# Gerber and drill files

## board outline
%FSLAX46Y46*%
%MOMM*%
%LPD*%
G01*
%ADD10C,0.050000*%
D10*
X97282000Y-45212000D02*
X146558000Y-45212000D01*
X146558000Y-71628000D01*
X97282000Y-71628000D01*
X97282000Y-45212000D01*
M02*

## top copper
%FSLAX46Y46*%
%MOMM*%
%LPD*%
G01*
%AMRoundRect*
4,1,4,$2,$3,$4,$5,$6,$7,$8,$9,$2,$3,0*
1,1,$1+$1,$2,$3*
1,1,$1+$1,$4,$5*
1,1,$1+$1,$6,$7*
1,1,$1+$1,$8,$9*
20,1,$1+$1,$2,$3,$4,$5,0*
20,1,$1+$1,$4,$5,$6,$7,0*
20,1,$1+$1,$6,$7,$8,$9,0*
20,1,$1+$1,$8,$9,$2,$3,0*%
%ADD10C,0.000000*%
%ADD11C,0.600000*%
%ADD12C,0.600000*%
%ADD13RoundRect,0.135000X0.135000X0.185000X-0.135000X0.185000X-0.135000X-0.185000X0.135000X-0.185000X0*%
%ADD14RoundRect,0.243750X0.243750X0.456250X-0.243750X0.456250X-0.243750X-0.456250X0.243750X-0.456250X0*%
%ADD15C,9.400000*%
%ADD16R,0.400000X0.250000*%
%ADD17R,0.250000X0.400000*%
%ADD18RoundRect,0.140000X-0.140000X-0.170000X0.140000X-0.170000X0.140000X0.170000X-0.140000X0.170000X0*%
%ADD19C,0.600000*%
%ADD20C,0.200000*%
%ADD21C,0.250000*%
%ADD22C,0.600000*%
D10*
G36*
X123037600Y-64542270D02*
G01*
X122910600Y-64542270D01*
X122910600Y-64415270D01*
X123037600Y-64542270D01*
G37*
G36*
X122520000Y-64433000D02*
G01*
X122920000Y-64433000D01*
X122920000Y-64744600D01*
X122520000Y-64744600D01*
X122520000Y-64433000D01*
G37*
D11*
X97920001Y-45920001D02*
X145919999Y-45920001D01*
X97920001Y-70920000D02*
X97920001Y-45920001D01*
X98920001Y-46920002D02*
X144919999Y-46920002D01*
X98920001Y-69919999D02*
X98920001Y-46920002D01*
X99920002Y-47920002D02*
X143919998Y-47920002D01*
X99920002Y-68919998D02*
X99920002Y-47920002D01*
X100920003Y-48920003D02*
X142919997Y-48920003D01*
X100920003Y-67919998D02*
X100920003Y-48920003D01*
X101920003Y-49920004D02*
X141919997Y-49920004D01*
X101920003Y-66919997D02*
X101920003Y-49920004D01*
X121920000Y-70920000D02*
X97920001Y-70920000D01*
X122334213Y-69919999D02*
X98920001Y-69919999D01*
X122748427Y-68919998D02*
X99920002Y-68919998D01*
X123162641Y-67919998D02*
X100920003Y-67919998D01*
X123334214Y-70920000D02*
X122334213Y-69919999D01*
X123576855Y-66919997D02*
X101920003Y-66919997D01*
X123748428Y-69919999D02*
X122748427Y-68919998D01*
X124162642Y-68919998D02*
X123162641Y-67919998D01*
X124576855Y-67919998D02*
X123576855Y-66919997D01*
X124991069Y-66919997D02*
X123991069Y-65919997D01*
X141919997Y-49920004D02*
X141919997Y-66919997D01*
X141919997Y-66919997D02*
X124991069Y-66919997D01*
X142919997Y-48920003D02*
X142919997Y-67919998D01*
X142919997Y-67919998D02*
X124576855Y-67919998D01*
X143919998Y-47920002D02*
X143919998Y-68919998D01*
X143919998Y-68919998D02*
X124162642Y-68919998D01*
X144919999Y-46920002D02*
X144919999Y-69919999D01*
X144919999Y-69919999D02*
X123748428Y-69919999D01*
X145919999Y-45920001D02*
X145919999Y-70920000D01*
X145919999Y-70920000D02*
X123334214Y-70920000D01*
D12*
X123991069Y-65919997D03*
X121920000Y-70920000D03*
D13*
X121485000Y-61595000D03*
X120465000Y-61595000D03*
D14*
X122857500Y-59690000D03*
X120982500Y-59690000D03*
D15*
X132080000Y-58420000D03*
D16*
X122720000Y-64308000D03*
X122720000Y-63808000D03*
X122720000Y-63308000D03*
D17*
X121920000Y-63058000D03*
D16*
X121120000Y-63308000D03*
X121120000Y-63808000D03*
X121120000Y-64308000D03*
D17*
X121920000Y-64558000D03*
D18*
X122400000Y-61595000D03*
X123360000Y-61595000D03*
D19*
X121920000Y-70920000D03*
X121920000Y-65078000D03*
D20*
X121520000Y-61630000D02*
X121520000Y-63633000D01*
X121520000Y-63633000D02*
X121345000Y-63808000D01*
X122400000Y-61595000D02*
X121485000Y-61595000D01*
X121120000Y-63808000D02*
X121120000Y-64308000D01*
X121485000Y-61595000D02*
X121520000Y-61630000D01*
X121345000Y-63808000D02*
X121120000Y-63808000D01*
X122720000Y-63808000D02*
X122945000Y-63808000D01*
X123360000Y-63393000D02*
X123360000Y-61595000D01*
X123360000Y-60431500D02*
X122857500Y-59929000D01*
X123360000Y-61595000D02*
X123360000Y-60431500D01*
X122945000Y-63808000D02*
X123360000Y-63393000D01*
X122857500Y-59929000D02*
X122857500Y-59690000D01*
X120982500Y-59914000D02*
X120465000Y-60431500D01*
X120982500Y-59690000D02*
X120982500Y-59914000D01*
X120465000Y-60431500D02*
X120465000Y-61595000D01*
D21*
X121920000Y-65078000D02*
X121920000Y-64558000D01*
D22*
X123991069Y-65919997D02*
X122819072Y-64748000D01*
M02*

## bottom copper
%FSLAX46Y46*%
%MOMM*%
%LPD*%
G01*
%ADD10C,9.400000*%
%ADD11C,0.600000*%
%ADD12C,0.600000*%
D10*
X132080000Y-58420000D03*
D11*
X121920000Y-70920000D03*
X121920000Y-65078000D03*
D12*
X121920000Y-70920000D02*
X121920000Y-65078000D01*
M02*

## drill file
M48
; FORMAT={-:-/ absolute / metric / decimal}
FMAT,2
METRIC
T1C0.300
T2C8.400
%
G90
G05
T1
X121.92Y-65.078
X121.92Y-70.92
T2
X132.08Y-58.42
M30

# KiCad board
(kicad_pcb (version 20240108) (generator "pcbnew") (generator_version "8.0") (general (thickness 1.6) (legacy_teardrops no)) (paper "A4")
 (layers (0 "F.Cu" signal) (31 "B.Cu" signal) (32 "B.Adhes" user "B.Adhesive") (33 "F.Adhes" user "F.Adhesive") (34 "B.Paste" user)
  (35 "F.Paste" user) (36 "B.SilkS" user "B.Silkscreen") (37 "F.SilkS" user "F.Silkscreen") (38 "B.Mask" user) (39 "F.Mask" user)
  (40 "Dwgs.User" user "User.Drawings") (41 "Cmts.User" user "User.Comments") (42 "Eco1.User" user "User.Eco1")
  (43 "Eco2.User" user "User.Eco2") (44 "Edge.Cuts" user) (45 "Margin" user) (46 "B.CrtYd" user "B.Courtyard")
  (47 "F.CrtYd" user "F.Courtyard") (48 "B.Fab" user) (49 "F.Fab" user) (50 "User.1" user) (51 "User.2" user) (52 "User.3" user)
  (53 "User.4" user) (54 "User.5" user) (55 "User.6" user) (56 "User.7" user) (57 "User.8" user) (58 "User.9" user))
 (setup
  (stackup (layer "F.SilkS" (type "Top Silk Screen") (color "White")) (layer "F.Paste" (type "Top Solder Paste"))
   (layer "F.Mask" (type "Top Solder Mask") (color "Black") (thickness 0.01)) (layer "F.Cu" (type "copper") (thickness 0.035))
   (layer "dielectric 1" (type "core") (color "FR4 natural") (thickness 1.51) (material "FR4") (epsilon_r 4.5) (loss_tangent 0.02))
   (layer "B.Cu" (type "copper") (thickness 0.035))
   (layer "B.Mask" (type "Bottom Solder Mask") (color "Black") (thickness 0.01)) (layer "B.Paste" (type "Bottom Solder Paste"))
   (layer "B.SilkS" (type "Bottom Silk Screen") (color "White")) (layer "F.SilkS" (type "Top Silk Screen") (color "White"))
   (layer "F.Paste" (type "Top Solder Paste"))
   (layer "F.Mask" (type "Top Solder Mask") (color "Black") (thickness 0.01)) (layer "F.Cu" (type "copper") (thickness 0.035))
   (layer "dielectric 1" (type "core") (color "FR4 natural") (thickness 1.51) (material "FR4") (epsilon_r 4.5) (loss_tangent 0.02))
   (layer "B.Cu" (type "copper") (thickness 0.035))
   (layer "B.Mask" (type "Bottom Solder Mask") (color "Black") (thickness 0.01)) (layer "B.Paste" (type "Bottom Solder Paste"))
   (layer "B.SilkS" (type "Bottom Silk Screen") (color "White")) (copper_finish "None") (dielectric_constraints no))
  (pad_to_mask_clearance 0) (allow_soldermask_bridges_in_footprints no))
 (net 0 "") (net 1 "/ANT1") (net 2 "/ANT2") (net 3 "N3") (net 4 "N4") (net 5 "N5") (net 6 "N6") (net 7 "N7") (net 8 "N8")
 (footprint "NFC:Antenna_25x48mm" (layer "F.Cu") (at 121.92 58.42)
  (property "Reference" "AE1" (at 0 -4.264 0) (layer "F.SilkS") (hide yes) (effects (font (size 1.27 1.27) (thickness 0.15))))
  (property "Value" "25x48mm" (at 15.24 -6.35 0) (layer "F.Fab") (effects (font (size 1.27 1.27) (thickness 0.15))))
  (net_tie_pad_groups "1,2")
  (fp_line (start -23.999999 -12.499999) (end 23.999999 -12.499999) (stroke (width 0.6) (type default)) (layer "F.Cu"))
  (fp_line (start -23.999999 12.5) (end -23.999999 -12.499999) (stroke (width 0.6) (type default)) (layer "F.Cu"))
  (fp_line (start -22.999999 -11.499998) (end 22.999999 -11.499998) (stroke (width 0.6) (type default)) (layer "F.Cu"))
  (fp_line (start -22.999999 11.499999) (end -22.999999 -11.499998) (stroke (width 0.6) (type default)) (layer "F.Cu"))
  (fp_line (start -21.999998 -10.499998) (end 21.999998 -10.499998) (stroke (width 0.6) (type default)) (layer "F.Cu"))
  (fp_line (start -21.999998 10.499998) (end -21.999998 -10.499998) (stroke (width 0.6) (type default)) (layer "F.Cu"))
  (fp_line (start -20.999997 -9.499997) (end 20.999997 -9.499997) (stroke (width 0.6) (type default)) (layer "F.Cu"))
  (fp_line (start -20.999997 9.499998) (end -20.999997 -9.499997) (stroke (width 0.6) (type default)) (layer "F.Cu"))
  (fp_line (start -19.999997 -8.499996) (end 19.999997 -8.499996) (stroke (width 0.6) (type default)) (layer "F.Cu"))
  (fp_line (start -19.999997 8.499997) (end -19.999997 -8.499996) (stroke (width 0.6) (type default)) (layer "F.Cu"))
  (fp_line (start 0 12.5) (end -23.999999 12.5) (stroke (width 0.6) (type default)) (layer "F.Cu"))
  (fp_line (start 0.414213 11.499999) (end -22.999999 11.499999) (stroke (width 0.6) (type default)) (layer "F.Cu"))
  (fp_line (start 0.828427 10.499998) (end -21.999998 10.499998) (stroke (width 0.6) (type default)) (layer "F.Cu"))
  (fp_line (start 1.242641 9.499998) (end -20.999997 9.499998) (stroke (width 0.6) (type default)) (layer "F.Cu"))
  (fp_line (start 1.414214 12.5) (end 0.414213 11.499999) (stroke (width 0.6) (type default)) (layer "F.Cu"))
  (fp_line (start 1.656855 8.499997) (end -19.999997 8.499997) (stroke (width 0.6) (type default)) (layer "F.Cu"))
  (fp_line (start 1.828428 11.499999) (end 0.828427 10.499998) (stroke (width 0.6) (type default)) (layer "F.Cu"))
  (fp_line (start 2.242642 10.499998) (end 1.242641 9.499998) (stroke (width 0.6) (type default)) (layer "F.Cu"))
  (fp_line (start 2.656855 9.499998) (end 1.656855 8.499997) (stroke (width 0.6) (type default)) (layer "F.Cu"))
  (fp_line (start 3.071069 8.499997) (end 2.071069 7.499997) (stroke (width 0.6) (type default)) (layer "F.Cu"))
  (fp_line (start 19.999997 -8.499996) (end 19.999997 8.499997) (stroke (width 0.6) (type default)) (layer "F.Cu"))
  (fp_line (start 19.999997 8.499997) (end 3.071069 8.499997) (stroke (width 0.6) (type default)) (layer "F.Cu"))
  (fp_line (start 20.999997 -9.499997) (end 20.999997 9.499998) (stroke (width 0.6) (type default)) (layer "F.Cu"))
  (fp_line (start 20.999997 9.499998) (end 2.656855 9.499998) (stroke (width 0.6) (type default)) (layer "F.Cu"))
  (fp_line (start 21.999998 -10.499998) (end 21.999998 10.499998) (stroke (width 0.6) (type default)) (layer "F.Cu"))
  (fp_line (start 21.999998 10.499998) (end 2.242642 10.499998) (stroke (width 0.6) (type default)) (layer "F.Cu"))
  (fp_line (start 22.999999 -11.499998) (end 22.999999 11.499999) (stroke (width 0.6) (type default)) (layer "F.Cu"))
  (fp_line (start 22.999999 11.499999) (end 1.828428 11.499999) (stroke (width 0.6) (type default)) (layer "F.Cu"))
  (fp_line (start 23.999999 -12.499999) (end 23.999999 12.5) (stroke (width 0.6) (type default)) (layer "F.Cu"))
  (fp_line (start 23.999999 12.5) (end 1.414214 12.5) (stroke (width 0.6) (type default)) (layer "F.Cu"))
  (pad "1" smd circle (at 2.071069 7.499997 90) (size 0.6 0.6) (layers "F.Cu") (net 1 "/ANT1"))
  (pad "2" smd circle (at 0 12.5) (size 0.6 0.6) (layers "F.Cu") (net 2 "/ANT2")))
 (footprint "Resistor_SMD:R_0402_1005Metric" (layer "F.Cu") (at 120.975 61.595 180)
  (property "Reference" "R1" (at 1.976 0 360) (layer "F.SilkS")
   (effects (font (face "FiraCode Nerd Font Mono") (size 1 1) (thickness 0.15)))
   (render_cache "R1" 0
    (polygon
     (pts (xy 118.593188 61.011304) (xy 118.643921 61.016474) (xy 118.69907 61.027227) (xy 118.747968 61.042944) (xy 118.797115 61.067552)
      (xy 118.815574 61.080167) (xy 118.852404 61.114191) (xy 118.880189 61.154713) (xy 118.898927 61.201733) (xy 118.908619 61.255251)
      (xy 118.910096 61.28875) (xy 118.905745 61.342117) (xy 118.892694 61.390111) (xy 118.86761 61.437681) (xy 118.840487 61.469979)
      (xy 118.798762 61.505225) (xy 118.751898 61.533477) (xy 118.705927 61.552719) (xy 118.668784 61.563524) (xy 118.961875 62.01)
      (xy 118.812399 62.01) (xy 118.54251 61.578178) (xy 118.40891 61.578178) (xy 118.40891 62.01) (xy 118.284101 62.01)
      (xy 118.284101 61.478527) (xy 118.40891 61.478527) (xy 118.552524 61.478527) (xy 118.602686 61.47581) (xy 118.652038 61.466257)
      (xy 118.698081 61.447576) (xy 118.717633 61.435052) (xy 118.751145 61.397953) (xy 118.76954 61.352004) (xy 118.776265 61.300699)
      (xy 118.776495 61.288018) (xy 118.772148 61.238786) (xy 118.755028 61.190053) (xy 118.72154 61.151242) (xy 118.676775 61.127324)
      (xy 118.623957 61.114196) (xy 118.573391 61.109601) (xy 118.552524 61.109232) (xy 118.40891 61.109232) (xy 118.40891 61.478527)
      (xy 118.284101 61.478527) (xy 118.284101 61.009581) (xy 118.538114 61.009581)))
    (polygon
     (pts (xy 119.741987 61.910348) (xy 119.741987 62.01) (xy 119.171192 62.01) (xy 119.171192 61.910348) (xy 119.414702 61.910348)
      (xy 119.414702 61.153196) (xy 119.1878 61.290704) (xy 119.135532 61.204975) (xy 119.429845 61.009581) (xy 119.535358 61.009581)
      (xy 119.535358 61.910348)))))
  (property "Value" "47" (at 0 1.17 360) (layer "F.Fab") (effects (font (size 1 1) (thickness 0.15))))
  (pad "1" smd roundrect (at -0.51 0 180) (size 0.54 0.64) (layers "F.Cu" "F.Paste" "F.Mask") (roundrect_rratio 0.25) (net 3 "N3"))
  (pad "2" smd roundrect (at 0.51 0 180) (size 0.54 0.64) (layers "F.Cu" "F.Paste" "F.Mask") (roundrect_rratio 0.25) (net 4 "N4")))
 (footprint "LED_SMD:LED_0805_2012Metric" (layer "F.Cu") (at 121.92 59.69 180)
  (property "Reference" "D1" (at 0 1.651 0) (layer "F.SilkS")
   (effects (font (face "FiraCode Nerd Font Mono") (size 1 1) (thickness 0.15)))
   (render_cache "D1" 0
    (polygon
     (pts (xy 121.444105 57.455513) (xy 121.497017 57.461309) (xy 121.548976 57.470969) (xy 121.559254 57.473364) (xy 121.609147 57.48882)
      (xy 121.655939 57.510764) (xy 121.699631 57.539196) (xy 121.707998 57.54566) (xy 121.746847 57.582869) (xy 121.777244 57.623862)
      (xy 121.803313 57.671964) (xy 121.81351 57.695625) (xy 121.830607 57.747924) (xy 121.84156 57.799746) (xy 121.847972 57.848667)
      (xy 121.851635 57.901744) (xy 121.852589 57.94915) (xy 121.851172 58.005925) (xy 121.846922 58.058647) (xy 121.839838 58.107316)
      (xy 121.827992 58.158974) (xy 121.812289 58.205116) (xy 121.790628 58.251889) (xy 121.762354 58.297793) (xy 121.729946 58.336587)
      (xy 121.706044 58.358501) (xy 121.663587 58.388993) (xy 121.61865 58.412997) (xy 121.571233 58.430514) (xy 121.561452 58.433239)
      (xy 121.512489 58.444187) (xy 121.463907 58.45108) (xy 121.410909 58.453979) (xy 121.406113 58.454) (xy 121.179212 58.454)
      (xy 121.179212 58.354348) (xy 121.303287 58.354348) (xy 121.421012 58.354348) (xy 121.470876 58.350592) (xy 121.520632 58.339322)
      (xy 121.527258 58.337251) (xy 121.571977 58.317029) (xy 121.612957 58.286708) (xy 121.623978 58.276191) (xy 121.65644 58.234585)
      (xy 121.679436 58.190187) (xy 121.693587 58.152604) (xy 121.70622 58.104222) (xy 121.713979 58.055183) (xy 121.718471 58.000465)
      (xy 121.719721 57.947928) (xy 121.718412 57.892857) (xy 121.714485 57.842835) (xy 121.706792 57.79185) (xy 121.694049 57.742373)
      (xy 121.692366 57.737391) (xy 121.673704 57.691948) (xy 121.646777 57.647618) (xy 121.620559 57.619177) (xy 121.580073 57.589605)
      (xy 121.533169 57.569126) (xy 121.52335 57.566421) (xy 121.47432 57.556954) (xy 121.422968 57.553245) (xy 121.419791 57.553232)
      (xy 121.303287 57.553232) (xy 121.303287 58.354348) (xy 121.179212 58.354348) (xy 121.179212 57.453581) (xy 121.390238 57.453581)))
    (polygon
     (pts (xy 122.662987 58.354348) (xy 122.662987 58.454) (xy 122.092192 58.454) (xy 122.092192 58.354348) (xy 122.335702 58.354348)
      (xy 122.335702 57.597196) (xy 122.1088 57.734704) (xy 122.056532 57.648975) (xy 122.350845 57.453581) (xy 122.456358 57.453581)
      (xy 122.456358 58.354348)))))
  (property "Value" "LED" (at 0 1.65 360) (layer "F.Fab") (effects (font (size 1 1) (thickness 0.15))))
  (pad "1" smd roundrect (at -0.9375 0 180) (size 0.975 1.4) (layers "F.Cu" "F.Paste" "F.Mask") (roundrect_rratio 0.25) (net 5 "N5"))
  (pad "2" smd roundrect (at 0.9375 0 180) (size 0.975 1.4) (layers "F.Cu" "F.Paste" "F.Mask") (roundrect_rratio 0.25) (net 4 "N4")))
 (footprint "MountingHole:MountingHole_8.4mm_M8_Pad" (layer "F.Cu") (at 132.08 58.42)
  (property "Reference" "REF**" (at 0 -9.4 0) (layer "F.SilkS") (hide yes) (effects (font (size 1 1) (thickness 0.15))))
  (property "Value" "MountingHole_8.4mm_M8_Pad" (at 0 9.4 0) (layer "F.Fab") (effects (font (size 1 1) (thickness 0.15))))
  (pad "1" thru_hole circle (at 0 0) (size 9.4 9.4) (drill 8.4) (layers "*.Cu" "*.Mask") (remove_unused_layers no)))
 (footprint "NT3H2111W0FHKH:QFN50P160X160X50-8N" (layer "F.Cu") (at 121.92 63.808 180)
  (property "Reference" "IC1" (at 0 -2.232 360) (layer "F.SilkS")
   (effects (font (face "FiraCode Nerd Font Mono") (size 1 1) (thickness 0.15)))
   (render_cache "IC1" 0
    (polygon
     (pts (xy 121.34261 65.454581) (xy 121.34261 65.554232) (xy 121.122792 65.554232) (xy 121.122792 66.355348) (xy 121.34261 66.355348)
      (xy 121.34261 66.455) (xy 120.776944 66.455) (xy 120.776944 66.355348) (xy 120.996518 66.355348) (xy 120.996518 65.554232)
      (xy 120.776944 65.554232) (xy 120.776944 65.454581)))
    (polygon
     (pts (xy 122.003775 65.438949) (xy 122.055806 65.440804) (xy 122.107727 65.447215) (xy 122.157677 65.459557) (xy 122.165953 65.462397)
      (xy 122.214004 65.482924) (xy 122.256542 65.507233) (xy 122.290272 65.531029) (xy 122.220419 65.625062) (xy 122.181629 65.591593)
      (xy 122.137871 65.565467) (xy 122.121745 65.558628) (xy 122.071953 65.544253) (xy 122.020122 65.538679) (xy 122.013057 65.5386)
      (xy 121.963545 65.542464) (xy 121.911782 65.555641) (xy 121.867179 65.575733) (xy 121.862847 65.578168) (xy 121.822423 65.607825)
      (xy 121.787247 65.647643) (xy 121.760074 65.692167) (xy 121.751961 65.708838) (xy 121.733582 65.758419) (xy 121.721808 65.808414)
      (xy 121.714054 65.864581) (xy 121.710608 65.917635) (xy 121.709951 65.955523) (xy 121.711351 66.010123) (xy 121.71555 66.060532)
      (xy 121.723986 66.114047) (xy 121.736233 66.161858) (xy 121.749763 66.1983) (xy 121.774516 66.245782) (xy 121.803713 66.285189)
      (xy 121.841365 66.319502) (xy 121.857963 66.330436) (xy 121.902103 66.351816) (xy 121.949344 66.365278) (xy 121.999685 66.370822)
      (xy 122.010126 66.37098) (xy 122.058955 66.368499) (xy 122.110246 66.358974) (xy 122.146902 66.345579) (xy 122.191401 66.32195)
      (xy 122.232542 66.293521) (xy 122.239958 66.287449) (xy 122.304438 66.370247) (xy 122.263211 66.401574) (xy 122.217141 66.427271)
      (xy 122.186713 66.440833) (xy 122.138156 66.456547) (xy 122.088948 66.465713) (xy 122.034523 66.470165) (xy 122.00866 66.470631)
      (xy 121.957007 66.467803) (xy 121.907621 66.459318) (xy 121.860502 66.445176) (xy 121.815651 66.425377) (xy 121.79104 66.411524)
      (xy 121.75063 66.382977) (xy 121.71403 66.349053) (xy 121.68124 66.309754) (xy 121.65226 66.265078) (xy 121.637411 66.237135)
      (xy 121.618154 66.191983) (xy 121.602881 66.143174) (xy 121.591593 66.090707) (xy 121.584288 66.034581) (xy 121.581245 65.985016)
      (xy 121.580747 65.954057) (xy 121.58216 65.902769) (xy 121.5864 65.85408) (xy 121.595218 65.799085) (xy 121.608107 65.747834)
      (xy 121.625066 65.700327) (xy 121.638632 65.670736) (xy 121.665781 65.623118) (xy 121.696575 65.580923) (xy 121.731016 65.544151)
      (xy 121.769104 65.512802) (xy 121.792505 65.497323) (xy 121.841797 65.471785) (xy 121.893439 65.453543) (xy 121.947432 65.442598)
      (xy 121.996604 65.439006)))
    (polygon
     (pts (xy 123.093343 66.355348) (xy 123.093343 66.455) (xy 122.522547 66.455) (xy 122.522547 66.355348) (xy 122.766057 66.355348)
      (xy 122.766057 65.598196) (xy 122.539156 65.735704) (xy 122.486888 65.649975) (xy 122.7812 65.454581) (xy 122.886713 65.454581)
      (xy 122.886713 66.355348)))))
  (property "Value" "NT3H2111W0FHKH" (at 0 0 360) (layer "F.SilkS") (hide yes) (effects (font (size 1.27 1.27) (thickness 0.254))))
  (pad "1" smd rect (at -0.8 -0.5 270) (size 0.25 0.4) (layers "F.Cu" "F.Paste" "F.Mask") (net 1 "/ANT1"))
  (pad "2" smd rect (at -0.8 0 270) (size 0.25 0.4) (layers "F.Cu" "F.Paste" "F.Mask") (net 5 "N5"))
  (pad "3" smd rect (at -0.8 0.5 270) (size 0.25 0.4) (layers "F.Cu" "F.Paste" "F.Mask") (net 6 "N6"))
  (pad "4" smd rect (at 0 0.75 180) (size 0.25 0.4) (layers "F.Cu" "F.Paste" "F.Mask") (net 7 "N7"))
  (pad "5" smd rect (at 0.8 0.5 270) (size 0.25 0.4) (layers "F.Cu" "F.Paste" "F.Mask") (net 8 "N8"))
  (pad "6" smd rect (at 0.8 0 270) (size 0.25 0.4) (layers "F.Cu" "F.Paste" "F.Mask") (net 3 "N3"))
  (pad "7" smd rect (at 0.8 -0.5 270) (size 0.25 0.4) (layers "F.Cu" "F.Paste" "F.Mask") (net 3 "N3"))
  (pad "8" smd rect (at 0 -0.75 180) (size 0.25 0.4) (layers "F.Cu" "F.Paste" "F.Mask") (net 2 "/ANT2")))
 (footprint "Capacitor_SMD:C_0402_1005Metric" (layer "F.Cu") (at 122.88 61.595)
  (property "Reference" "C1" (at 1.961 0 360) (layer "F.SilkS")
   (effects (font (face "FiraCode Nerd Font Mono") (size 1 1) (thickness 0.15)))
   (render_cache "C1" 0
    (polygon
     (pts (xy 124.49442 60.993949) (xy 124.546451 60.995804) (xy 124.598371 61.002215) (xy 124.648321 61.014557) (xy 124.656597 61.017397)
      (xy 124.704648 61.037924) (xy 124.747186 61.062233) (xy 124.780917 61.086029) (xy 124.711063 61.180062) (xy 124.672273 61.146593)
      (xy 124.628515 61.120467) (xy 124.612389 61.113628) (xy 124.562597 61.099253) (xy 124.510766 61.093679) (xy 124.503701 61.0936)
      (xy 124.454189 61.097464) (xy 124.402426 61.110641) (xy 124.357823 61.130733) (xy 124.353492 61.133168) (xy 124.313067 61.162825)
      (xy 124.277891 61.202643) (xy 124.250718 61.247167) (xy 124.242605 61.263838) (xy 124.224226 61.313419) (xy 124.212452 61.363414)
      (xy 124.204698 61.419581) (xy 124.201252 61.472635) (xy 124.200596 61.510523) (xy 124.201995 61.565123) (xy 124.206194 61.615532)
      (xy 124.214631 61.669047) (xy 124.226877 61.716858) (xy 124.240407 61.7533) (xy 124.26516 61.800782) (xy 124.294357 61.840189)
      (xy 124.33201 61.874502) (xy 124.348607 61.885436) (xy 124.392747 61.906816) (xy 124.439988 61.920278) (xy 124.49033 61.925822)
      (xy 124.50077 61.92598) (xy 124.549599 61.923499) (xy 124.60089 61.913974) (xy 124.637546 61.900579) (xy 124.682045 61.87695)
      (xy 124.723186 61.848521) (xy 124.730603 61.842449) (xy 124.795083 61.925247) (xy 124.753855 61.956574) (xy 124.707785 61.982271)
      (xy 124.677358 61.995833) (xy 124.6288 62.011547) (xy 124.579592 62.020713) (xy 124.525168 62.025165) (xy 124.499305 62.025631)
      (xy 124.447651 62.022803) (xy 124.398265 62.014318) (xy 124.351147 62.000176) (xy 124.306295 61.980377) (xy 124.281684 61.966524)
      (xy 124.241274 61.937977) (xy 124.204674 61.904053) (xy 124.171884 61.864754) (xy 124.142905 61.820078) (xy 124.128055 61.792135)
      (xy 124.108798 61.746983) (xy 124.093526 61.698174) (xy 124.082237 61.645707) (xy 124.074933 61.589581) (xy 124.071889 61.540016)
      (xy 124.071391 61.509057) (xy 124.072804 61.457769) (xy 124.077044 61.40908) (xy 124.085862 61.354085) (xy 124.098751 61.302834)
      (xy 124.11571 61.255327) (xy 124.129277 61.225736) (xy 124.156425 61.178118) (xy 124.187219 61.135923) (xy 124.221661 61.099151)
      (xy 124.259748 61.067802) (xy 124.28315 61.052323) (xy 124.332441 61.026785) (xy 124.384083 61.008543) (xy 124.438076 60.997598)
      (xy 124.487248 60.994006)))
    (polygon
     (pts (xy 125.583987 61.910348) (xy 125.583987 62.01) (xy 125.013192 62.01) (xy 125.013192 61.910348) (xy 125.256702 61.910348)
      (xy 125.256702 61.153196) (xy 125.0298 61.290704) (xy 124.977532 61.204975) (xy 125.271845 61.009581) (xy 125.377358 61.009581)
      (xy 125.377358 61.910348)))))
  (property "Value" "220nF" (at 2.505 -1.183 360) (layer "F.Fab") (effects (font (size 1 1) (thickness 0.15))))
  (pad "1" smd roundrect (at -0.48 0) (size 0.56 0.62) (layers "F.Cu" "F.Paste" "F.Mask") (roundrect_rratio 0.25) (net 3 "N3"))
  (pad "2" smd roundrect (at 0.48 0) (size 0.56 0.62) (layers "F.Cu" "F.Paste" "F.Mask") (roundrect_rratio 0.25) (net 5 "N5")))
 (gr_poly
  (pts (xy 122.9106 64.41527) (xy 123.0376 64.54227) (xy 122.9106 64.54227)) (stroke (width 0) (type solid)) (fill solid) (layer "F.Cu")
  (net 1))
 (gr_rect (start 122.52 64.433) (end 122.92 64.7446) (stroke (width 0) (type default)) (fill solid) (layer "F.Cu") (net 1))
 (gr_rect (start 97.282 45.212) (end 146.558 71.628) (stroke (width 0.05) (type default)) (fill none) (layer "Edge.Cuts"))
 (segment (start 121.52 61.63) (end 121.52 63.633) (width 0.2) (layer "F.Cu") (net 3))
 (segment (start 121.52 63.633) (end 121.345 63.808) (width 0.2) (layer "F.Cu") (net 3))
 (segment (start 122.4 61.595) (end 121.485 61.595) (width 0.2) (layer "F.Cu") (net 3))
 (segment (start 121.12 63.808) (end 121.12 64.308) (width 0.2) (layer "F.Cu") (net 3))
 (segment (start 121.485 61.595) (end 121.52 61.63) (width 0.2) (layer "F.Cu") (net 3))
 (segment (start 121.345 63.808) (end 121.12 63.808) (width 0.2) (layer "F.Cu") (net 3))
 (segment (start 122.72 63.808) (end 122.945 63.808) (width 0.2) (layer "F.Cu") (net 5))
 (segment (start 123.36 63.393) (end 123.36 61.595) (width 0.2) (layer "F.Cu") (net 5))
 (segment (start 123.36 60.4315) (end 122.8575 59.929) (width 0.2) (layer "F.Cu") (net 5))
 (segment (start 123.36 61.595) (end 123.36 60.4315) (width 0.2) (layer "F.Cu") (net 5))
 (segment (start 122.945 63.808) (end 123.36 63.393) (width 0.2) (layer "F.Cu") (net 5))
 (segment (start 122.8575 59.929) (end 122.8575 59.69) (width 0.2) (layer "F.Cu") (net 5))
 (segment (start 120.9825 59.914) (end 120.465 60.4315) (width 0.2) (layer "F.Cu") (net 4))
 (segment (start 120.9825 59.69) (end 120.9825 59.914) (width 0.2) (layer "F.Cu") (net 4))
 (segment (start 120.465 60.4315) (end 120.465 61.595) (width 0.2) (layer "F.Cu") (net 4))
 (segment (start 121.92 65.078) (end 121.92 64.558) (width 0.25) (layer "F.Cu") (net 2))
 (via (at 121.92 70.92) (size 0.6) (drill 0.3) (layers "F.Cu" "B.Cu") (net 2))
 (via (at 121.92 65.078) (size 0.6) (drill 0.3) (layers "F.Cu" "B.Cu") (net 2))
 (segment (start 121.92 70.92) (end 121.92 65.078) (width 0.6) (layer "B.Cu") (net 2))
 (segment (start 123.991069 65.919997) (end 122.819072 64.748) (width 0.6) (layer "F.Cu") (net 1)))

